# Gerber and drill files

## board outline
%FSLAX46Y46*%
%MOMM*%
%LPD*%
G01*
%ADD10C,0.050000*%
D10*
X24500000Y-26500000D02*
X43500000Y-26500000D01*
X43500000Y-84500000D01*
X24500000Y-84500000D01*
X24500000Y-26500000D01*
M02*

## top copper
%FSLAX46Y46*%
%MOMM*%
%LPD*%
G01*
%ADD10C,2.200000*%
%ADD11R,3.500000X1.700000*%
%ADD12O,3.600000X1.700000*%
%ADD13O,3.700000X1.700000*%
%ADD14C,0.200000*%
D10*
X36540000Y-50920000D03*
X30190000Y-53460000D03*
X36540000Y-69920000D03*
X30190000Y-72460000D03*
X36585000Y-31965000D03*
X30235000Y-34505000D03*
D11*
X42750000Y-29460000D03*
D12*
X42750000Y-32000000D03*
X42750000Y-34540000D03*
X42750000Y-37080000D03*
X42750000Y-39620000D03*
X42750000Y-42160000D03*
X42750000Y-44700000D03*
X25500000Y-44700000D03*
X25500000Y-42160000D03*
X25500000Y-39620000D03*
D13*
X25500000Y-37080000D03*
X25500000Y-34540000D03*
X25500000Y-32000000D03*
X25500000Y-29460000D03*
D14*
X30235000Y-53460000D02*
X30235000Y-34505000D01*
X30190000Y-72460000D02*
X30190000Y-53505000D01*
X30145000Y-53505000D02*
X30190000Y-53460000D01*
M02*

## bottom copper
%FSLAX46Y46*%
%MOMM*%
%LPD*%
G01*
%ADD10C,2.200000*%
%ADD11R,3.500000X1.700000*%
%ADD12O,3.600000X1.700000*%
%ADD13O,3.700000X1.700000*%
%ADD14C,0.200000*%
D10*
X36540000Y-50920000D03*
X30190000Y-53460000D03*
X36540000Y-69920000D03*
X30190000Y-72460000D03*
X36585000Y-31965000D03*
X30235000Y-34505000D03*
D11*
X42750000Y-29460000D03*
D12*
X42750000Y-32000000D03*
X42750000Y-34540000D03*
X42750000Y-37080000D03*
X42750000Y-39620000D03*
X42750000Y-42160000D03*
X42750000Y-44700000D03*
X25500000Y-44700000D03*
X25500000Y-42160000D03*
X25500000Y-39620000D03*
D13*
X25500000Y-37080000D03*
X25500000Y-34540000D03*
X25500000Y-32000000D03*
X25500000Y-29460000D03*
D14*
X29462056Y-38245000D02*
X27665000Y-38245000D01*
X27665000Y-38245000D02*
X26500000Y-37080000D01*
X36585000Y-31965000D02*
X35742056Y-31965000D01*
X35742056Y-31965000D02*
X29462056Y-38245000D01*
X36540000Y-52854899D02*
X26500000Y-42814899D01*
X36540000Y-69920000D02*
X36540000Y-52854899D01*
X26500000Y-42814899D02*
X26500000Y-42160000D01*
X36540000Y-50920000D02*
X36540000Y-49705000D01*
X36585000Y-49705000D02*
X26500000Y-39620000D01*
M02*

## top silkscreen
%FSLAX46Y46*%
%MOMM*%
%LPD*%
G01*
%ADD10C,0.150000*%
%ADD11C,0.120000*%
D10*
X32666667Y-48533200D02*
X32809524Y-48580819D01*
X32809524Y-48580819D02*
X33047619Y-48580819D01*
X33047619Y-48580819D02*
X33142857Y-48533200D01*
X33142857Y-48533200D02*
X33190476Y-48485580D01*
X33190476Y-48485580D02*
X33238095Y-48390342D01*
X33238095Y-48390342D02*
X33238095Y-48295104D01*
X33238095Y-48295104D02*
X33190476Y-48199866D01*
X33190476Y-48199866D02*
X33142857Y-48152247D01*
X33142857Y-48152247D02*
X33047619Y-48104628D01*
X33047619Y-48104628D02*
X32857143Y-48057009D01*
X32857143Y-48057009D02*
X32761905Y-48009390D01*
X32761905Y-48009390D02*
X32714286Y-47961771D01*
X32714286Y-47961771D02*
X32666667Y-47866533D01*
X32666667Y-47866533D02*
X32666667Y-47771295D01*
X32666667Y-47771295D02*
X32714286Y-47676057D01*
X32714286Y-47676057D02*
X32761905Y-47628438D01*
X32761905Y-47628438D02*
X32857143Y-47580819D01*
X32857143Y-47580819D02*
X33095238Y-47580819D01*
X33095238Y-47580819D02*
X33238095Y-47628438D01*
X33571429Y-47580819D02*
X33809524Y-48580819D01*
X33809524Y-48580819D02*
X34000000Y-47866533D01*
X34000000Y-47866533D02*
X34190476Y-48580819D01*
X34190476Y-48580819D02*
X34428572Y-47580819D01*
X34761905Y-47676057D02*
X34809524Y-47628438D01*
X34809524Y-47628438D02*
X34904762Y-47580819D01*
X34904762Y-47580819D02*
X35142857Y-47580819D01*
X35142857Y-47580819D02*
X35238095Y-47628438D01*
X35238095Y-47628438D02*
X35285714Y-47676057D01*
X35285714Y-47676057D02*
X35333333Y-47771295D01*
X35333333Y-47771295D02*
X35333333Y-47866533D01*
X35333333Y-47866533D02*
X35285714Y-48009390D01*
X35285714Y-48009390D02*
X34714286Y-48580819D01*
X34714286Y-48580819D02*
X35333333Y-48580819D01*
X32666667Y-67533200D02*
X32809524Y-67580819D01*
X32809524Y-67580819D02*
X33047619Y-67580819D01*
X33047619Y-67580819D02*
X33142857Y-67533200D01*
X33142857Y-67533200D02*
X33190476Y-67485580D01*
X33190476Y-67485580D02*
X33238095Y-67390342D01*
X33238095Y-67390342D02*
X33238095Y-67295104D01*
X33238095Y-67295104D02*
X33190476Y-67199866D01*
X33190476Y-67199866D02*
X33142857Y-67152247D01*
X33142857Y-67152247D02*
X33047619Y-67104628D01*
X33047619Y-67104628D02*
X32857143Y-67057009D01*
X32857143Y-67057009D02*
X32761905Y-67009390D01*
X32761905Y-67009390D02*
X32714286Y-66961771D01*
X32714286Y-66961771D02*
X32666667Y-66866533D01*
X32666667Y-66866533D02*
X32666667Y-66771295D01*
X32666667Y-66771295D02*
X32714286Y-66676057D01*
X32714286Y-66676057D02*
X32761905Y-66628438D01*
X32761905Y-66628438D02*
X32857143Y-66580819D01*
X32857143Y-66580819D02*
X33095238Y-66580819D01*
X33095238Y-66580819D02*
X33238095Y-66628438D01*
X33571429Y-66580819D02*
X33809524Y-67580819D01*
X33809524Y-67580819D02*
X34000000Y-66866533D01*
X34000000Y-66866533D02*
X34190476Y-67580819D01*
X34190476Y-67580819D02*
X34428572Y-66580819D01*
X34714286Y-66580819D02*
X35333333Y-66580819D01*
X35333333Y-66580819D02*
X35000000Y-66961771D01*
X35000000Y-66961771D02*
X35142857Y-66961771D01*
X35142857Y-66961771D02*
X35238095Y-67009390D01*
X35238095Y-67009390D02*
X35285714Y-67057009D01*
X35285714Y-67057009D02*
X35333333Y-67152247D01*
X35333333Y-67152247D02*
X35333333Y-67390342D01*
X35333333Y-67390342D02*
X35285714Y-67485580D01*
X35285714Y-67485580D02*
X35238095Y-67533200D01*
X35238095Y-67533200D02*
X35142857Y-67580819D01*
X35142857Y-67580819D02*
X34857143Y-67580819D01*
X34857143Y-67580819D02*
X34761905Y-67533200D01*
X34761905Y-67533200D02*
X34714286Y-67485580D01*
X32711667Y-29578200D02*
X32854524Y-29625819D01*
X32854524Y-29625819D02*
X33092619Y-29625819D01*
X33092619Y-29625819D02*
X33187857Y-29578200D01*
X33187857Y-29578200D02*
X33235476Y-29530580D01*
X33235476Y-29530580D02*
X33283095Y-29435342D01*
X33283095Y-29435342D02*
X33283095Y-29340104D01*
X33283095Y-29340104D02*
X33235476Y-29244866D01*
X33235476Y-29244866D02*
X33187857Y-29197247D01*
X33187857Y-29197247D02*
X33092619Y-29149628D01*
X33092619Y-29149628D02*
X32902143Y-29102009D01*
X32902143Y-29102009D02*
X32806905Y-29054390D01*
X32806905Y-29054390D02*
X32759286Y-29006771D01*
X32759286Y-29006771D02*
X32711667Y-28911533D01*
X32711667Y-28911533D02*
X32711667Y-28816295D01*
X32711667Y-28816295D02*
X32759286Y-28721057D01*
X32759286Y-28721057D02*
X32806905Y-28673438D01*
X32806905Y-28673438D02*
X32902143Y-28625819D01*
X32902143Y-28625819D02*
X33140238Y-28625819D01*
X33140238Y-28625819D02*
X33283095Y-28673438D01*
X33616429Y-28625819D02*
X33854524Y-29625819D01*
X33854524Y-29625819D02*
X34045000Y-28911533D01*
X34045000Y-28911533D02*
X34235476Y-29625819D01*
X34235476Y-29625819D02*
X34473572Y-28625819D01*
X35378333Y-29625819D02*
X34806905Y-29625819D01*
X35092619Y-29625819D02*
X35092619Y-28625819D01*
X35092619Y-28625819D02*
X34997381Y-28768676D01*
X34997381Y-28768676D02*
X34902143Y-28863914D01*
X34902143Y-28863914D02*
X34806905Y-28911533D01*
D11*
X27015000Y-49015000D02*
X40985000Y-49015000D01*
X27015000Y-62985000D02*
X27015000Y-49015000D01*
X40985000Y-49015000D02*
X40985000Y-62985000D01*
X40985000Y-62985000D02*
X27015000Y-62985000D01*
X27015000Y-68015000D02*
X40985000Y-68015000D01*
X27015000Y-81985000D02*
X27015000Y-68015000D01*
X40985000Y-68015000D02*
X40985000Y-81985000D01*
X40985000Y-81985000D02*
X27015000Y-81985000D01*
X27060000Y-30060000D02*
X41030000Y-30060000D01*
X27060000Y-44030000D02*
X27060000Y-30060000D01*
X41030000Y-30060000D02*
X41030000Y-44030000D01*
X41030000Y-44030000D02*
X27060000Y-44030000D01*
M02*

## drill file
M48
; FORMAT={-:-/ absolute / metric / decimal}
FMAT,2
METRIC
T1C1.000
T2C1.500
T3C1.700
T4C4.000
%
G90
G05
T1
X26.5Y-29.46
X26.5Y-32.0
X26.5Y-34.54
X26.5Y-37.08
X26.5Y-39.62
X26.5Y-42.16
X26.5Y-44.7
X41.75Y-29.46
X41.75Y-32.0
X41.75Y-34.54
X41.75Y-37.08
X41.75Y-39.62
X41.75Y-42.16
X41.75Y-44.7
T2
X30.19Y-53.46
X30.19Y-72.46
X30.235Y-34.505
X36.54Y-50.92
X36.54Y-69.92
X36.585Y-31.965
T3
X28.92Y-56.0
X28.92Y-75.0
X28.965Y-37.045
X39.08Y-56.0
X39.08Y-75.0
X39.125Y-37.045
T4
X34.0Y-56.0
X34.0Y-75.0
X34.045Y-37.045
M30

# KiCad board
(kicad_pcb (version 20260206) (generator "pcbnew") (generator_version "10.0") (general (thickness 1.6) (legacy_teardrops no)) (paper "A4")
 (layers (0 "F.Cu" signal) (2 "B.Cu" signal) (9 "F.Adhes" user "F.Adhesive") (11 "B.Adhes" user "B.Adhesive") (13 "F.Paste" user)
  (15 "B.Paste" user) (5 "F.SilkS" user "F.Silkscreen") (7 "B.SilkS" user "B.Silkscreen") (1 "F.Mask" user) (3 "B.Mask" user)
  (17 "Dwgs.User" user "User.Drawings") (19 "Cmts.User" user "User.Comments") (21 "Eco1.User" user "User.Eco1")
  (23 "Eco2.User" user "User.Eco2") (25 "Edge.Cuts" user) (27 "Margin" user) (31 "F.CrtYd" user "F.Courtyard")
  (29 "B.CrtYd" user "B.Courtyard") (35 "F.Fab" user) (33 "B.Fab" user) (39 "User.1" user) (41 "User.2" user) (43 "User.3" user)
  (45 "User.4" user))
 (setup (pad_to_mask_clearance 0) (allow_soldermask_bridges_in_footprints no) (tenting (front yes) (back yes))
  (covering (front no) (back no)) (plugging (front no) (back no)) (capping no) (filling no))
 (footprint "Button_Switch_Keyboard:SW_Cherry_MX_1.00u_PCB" (layer "F.Cu") (at 36.54 50.92)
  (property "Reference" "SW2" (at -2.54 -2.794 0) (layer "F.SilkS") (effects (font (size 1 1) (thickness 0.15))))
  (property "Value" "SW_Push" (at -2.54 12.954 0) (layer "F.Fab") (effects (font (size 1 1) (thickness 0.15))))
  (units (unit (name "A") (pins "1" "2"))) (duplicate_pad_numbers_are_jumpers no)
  (fp_line (start -9.525 -1.905) (end 4.445 -1.905) (stroke (width 0.12) (type solid)) (layer "F.SilkS"))
  (fp_line (start -9.525 12.065) (end -9.525 -1.905) (stroke (width 0.12) (type solid)) (layer "F.SilkS"))
  (fp_line (start 4.445 -1.905) (end 4.445 12.065) (stroke (width 0.12) (type solid)) (layer "F.SilkS"))
  (fp_line (start 4.445 12.065) (end -9.525 12.065) (stroke (width 0.12) (type solid)) (layer "F.SilkS"))
  (pad "" np_thru_hole circle (at -7.62 5.08) (size 1.7 1.7) (drill 1.7) (layers "*.Cu" "*.Mask"))
  (pad "" np_thru_hole circle (at -2.54 5.08) (size 4 4) (drill 4) (layers "*.Cu" "*.Mask"))
  (pad "" np_thru_hole circle (at 2.54 5.08) (size 1.7 1.7) (drill 1.7) (layers "*.Cu" "*.Mask"))
  (pad "1" thru_hole circle (at 0 0) (size 2.2 2.2) (drill 1.5) (layers "*.Cu" "*.Mask") (remove_unused_layers no)
   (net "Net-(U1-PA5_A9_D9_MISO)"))
  (pad "2" thru_hole circle (at -6.35 2.54) (size 2.2 2.2) (drill 1.5) (layers "*.Cu" "*.Mask") (remove_unused_layers no) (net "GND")))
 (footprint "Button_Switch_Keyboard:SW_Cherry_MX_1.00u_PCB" (layer "F.Cu") (at 36.54 69.92)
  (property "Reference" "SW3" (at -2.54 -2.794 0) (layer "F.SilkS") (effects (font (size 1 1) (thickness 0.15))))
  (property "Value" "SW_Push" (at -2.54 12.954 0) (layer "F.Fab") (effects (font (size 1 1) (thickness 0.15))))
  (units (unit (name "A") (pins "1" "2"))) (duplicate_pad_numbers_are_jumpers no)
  (fp_line (start -9.525 -1.905) (end 4.445 -1.905) (stroke (width 0.12) (type solid)) (layer "F.SilkS"))
  (fp_line (start -9.525 12.065) (end -9.525 -1.905) (stroke (width 0.12) (type solid)) (layer "F.SilkS"))
  (fp_line (start 4.445 -1.905) (end 4.445 12.065) (stroke (width 0.12) (type solid)) (layer "F.SilkS"))
  (fp_line (start 4.445 12.065) (end -9.525 12.065) (stroke (width 0.12) (type solid)) (layer "F.SilkS"))
  (pad "" np_thru_hole circle (at -7.62 5.08) (size 1.7 1.7) (drill 1.7) (layers "*.Cu" "*.Mask"))
  (pad "" np_thru_hole circle (at -2.54 5.08) (size 4 4) (drill 4) (layers "*.Cu" "*.Mask"))
  (pad "" np_thru_hole circle (at 2.54 5.08) (size 1.7 1.7) (drill 1.7) (layers "*.Cu" "*.Mask"))
  (pad "1" thru_hole circle (at 0 0) (size 2.2 2.2) (drill 1.5) (layers "*.Cu" "*.Mask") (remove_unused_layers no)
   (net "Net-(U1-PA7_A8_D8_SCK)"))
  (pad "2" thru_hole circle (at -6.35 2.54) (size 2.2 2.2) (drill 1.5) (layers "*.Cu" "*.Mask") (remove_unused_layers no) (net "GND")))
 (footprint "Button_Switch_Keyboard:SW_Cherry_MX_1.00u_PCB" (layer "F.Cu") (at 36.585 31.965)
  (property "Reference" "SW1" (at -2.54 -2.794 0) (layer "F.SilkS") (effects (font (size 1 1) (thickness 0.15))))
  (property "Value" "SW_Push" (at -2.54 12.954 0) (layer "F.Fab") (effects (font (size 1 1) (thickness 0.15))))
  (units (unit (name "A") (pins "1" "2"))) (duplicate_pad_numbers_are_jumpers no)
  (fp_line (start -9.525 -1.905) (end 4.445 -1.905) (stroke (width 0.12) (type solid)) (layer "F.SilkS"))
  (fp_line (start -9.525 12.065) (end -9.525 -1.905) (stroke (width 0.12) (type solid)) (layer "F.SilkS"))
  (fp_line (start 4.445 -1.905) (end 4.445 12.065) (stroke (width 0.12) (type solid)) (layer "F.SilkS"))
  (fp_line (start 4.445 12.065) (end -9.525 12.065) (stroke (width 0.12) (type solid)) (layer "F.SilkS"))
  (pad "" np_thru_hole circle (at -7.62 5.08) (size 1.7 1.7) (drill 1.7) (layers "*.Cu" "*.Mask"))
  (pad "" np_thru_hole circle (at -2.54 5.08) (size 4 4) (drill 4) (layers "*.Cu" "*.Mask"))
  (pad "" np_thru_hole circle (at 2.54 5.08) (size 1.7 1.7) (drill 1.7) (layers "*.Cu" "*.Mask"))
  (pad "1" thru_hole circle (at 0 0) (size 2.2 2.2) (drill 1.5) (layers "*.Cu" "*.Mask") (remove_unused_layers no)
   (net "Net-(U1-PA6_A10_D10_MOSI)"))
  (pad "2" thru_hole circle (at -6.35 2.54) (size 2.2 2.2) (drill 1.5) (layers "*.Cu" "*.Mask") (remove_unused_layers no) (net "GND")))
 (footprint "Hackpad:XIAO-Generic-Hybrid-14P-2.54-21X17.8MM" (layer "B.Cu") (at 34.125 37.08 180)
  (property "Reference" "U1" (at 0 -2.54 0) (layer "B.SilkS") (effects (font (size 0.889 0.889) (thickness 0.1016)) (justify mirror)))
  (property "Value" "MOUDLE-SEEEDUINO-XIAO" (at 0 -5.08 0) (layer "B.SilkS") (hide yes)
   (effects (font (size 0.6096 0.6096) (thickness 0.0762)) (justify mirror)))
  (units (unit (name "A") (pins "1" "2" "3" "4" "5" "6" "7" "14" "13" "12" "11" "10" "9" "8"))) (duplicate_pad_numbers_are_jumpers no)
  (pad "1" thru_hole rect (at -7.625 7.62 180) (size 3.5 1.7) (drill 1 (offset -1 0)) (layers "*.Cu" "*.Mask") (remove_unused_layers no)
   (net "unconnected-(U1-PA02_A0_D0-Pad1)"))
  (pad "2" thru_hole oval (at -7.625 5.08 180) (size 3.6 1.7) (drill 1 (offset -1 0)) (layers "*.Cu" "*.Mask") (remove_unused_layers no)
   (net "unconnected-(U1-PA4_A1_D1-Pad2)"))
  (pad "3" thru_hole oval (at -7.625 2.54 180) (size 3.6 1.7) (drill 1 (offset -1 0)) (layers "*.Cu" "*.Mask") (remove_unused_layers no)
   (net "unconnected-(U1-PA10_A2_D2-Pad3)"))
  (pad "4" thru_hole oval (at -7.625 0 180) (size 3.6 1.7) (drill 1 (offset -1 0)) (layers "*.Cu" "*.Mask") (remove_unused_layers no)
   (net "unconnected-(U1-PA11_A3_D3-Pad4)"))
  (pad "5" thru_hole oval (at -7.625 -2.54 180) (size 3.6 1.7) (drill 1 (offset -1 0)) (layers "*.Cu" "*.Mask") (remove_unused_layers no)
   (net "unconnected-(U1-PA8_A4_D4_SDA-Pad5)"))
  (pad "6" thru_hole oval (at -7.625 -5.08) (size 3.6 1.7) (drill 1 (offset 1 0)) (layers "*.Cu" "*.Mask") (remove_unused_layers no)
   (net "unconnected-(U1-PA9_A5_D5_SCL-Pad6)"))
  (pad "7" thru_hole oval (at -7.625 -7.62 180) (size 3.6 1.7) (drill 1 (offset -1 0)) (layers "*.Cu" "*.Mask") (remove_unused_layers no)
   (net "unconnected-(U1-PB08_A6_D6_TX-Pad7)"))
  (pad "8" thru_hole oval (at 7.625 -7.62 180) (size 3.6 1.7) (drill 1 (offset 1 0)) (layers "*.Cu" "*.Mask") (remove_unused_layers no)
   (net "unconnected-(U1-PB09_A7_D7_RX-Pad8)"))
  (pad "9" thru_hole oval (at 7.625 -5.08 180) (size 3.6 1.7) (drill 1 (offset 1 0)) (layers "*.Cu" "*.Mask") (remove_unused_layers no)
   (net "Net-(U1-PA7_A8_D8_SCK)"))
  (pad "10" thru_hole oval (at 7.625 -2.54 180) (size 3.6 1.7) (drill 1 (offset 1 0)) (layers "*.Cu" "*.Mask") (remove_unused_layers no)
   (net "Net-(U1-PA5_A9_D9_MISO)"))
  (pad "11" thru_hole oval (at 7.625 0 180) (size 3.7 1.7) (drill 1 (offset 1 0)) (layers "*.Cu" "*.Mask") (remove_unused_layers no)
   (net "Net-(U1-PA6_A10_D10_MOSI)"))
  (pad "12" thru_hole oval (at 7.625 2.54 180) (size 3.7 1.7) (drill 1 (offset 1 0)) (layers "*.Cu" "*.Mask") (remove_unused_layers no)
   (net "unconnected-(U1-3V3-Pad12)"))
  (pad "13" thru_hole oval (at 7.625 5.08 180) (size 3.7 1.7) (drill 1 (offset 1 0)) (layers "*.Cu" "*.Mask") (remove_unused_layers no)
   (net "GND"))
  (pad "14" thru_hole oval (at 7.625 7.62 180) (size 3.7 1.7) (drill 1 (offset 1 0)) (layers "*.Cu" "*.Mask") (remove_unused_layers no)
   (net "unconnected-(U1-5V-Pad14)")))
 (gr_rect (start 24.5 26.5) (end 43.5 84.5) (stroke (width 0.05) (type default)) (fill no) (layer "Edge.Cuts"))
 (segment (start 29.462056 38.245) (end 27.665 38.245) (width 0.2) (layer "B.Cu") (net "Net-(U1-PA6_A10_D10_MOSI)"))
 (segment (start 27.665 38.245) (end 26.5 37.08) (width 0.2) (layer "B.Cu") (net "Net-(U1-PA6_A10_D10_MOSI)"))
 (segment (start 36.585 31.965) (end 35.742056 31.965) (width 0.2) (layer "B.Cu") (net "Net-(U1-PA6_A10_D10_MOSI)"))
 (segment (start 35.742056 31.965) (end 29.462056 38.245) (width 0.2) (layer "B.Cu") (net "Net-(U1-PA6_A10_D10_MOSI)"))
 (segment (start 30.235 53.46) (end 30.235 34.505) (width 0.2) (layer "F.Cu") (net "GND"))
 (segment (start 30.19 72.46) (end 30.19 53.505) (width 0.2) (layer "F.Cu") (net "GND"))
 (segment (start 30.145 53.505) (end 30.19 53.46) (width 0.2) (layer "F.Cu") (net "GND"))
 (segment (start 36.54 52.854899) (end 26.5 42.814899) (width 0.2) (layer "B.Cu") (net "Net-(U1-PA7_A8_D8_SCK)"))
 (segment (start 36.54 69.92) (end 36.54 52.854899) (width 0.2) (layer "B.Cu") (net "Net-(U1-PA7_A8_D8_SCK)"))
 (segment (start 26.5 42.814899) (end 26.5 42.16) (width 0.2) (layer "B.Cu") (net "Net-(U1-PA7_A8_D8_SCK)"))
 (segment (start 36.54 50.92) (end 36.54 49.705) (width 0.2) (layer "B.Cu") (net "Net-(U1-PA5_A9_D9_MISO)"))
 (segment (start 36.585 49.705) (end 26.5 39.62) (width 0.2) (layer "B.Cu") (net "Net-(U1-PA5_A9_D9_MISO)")))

